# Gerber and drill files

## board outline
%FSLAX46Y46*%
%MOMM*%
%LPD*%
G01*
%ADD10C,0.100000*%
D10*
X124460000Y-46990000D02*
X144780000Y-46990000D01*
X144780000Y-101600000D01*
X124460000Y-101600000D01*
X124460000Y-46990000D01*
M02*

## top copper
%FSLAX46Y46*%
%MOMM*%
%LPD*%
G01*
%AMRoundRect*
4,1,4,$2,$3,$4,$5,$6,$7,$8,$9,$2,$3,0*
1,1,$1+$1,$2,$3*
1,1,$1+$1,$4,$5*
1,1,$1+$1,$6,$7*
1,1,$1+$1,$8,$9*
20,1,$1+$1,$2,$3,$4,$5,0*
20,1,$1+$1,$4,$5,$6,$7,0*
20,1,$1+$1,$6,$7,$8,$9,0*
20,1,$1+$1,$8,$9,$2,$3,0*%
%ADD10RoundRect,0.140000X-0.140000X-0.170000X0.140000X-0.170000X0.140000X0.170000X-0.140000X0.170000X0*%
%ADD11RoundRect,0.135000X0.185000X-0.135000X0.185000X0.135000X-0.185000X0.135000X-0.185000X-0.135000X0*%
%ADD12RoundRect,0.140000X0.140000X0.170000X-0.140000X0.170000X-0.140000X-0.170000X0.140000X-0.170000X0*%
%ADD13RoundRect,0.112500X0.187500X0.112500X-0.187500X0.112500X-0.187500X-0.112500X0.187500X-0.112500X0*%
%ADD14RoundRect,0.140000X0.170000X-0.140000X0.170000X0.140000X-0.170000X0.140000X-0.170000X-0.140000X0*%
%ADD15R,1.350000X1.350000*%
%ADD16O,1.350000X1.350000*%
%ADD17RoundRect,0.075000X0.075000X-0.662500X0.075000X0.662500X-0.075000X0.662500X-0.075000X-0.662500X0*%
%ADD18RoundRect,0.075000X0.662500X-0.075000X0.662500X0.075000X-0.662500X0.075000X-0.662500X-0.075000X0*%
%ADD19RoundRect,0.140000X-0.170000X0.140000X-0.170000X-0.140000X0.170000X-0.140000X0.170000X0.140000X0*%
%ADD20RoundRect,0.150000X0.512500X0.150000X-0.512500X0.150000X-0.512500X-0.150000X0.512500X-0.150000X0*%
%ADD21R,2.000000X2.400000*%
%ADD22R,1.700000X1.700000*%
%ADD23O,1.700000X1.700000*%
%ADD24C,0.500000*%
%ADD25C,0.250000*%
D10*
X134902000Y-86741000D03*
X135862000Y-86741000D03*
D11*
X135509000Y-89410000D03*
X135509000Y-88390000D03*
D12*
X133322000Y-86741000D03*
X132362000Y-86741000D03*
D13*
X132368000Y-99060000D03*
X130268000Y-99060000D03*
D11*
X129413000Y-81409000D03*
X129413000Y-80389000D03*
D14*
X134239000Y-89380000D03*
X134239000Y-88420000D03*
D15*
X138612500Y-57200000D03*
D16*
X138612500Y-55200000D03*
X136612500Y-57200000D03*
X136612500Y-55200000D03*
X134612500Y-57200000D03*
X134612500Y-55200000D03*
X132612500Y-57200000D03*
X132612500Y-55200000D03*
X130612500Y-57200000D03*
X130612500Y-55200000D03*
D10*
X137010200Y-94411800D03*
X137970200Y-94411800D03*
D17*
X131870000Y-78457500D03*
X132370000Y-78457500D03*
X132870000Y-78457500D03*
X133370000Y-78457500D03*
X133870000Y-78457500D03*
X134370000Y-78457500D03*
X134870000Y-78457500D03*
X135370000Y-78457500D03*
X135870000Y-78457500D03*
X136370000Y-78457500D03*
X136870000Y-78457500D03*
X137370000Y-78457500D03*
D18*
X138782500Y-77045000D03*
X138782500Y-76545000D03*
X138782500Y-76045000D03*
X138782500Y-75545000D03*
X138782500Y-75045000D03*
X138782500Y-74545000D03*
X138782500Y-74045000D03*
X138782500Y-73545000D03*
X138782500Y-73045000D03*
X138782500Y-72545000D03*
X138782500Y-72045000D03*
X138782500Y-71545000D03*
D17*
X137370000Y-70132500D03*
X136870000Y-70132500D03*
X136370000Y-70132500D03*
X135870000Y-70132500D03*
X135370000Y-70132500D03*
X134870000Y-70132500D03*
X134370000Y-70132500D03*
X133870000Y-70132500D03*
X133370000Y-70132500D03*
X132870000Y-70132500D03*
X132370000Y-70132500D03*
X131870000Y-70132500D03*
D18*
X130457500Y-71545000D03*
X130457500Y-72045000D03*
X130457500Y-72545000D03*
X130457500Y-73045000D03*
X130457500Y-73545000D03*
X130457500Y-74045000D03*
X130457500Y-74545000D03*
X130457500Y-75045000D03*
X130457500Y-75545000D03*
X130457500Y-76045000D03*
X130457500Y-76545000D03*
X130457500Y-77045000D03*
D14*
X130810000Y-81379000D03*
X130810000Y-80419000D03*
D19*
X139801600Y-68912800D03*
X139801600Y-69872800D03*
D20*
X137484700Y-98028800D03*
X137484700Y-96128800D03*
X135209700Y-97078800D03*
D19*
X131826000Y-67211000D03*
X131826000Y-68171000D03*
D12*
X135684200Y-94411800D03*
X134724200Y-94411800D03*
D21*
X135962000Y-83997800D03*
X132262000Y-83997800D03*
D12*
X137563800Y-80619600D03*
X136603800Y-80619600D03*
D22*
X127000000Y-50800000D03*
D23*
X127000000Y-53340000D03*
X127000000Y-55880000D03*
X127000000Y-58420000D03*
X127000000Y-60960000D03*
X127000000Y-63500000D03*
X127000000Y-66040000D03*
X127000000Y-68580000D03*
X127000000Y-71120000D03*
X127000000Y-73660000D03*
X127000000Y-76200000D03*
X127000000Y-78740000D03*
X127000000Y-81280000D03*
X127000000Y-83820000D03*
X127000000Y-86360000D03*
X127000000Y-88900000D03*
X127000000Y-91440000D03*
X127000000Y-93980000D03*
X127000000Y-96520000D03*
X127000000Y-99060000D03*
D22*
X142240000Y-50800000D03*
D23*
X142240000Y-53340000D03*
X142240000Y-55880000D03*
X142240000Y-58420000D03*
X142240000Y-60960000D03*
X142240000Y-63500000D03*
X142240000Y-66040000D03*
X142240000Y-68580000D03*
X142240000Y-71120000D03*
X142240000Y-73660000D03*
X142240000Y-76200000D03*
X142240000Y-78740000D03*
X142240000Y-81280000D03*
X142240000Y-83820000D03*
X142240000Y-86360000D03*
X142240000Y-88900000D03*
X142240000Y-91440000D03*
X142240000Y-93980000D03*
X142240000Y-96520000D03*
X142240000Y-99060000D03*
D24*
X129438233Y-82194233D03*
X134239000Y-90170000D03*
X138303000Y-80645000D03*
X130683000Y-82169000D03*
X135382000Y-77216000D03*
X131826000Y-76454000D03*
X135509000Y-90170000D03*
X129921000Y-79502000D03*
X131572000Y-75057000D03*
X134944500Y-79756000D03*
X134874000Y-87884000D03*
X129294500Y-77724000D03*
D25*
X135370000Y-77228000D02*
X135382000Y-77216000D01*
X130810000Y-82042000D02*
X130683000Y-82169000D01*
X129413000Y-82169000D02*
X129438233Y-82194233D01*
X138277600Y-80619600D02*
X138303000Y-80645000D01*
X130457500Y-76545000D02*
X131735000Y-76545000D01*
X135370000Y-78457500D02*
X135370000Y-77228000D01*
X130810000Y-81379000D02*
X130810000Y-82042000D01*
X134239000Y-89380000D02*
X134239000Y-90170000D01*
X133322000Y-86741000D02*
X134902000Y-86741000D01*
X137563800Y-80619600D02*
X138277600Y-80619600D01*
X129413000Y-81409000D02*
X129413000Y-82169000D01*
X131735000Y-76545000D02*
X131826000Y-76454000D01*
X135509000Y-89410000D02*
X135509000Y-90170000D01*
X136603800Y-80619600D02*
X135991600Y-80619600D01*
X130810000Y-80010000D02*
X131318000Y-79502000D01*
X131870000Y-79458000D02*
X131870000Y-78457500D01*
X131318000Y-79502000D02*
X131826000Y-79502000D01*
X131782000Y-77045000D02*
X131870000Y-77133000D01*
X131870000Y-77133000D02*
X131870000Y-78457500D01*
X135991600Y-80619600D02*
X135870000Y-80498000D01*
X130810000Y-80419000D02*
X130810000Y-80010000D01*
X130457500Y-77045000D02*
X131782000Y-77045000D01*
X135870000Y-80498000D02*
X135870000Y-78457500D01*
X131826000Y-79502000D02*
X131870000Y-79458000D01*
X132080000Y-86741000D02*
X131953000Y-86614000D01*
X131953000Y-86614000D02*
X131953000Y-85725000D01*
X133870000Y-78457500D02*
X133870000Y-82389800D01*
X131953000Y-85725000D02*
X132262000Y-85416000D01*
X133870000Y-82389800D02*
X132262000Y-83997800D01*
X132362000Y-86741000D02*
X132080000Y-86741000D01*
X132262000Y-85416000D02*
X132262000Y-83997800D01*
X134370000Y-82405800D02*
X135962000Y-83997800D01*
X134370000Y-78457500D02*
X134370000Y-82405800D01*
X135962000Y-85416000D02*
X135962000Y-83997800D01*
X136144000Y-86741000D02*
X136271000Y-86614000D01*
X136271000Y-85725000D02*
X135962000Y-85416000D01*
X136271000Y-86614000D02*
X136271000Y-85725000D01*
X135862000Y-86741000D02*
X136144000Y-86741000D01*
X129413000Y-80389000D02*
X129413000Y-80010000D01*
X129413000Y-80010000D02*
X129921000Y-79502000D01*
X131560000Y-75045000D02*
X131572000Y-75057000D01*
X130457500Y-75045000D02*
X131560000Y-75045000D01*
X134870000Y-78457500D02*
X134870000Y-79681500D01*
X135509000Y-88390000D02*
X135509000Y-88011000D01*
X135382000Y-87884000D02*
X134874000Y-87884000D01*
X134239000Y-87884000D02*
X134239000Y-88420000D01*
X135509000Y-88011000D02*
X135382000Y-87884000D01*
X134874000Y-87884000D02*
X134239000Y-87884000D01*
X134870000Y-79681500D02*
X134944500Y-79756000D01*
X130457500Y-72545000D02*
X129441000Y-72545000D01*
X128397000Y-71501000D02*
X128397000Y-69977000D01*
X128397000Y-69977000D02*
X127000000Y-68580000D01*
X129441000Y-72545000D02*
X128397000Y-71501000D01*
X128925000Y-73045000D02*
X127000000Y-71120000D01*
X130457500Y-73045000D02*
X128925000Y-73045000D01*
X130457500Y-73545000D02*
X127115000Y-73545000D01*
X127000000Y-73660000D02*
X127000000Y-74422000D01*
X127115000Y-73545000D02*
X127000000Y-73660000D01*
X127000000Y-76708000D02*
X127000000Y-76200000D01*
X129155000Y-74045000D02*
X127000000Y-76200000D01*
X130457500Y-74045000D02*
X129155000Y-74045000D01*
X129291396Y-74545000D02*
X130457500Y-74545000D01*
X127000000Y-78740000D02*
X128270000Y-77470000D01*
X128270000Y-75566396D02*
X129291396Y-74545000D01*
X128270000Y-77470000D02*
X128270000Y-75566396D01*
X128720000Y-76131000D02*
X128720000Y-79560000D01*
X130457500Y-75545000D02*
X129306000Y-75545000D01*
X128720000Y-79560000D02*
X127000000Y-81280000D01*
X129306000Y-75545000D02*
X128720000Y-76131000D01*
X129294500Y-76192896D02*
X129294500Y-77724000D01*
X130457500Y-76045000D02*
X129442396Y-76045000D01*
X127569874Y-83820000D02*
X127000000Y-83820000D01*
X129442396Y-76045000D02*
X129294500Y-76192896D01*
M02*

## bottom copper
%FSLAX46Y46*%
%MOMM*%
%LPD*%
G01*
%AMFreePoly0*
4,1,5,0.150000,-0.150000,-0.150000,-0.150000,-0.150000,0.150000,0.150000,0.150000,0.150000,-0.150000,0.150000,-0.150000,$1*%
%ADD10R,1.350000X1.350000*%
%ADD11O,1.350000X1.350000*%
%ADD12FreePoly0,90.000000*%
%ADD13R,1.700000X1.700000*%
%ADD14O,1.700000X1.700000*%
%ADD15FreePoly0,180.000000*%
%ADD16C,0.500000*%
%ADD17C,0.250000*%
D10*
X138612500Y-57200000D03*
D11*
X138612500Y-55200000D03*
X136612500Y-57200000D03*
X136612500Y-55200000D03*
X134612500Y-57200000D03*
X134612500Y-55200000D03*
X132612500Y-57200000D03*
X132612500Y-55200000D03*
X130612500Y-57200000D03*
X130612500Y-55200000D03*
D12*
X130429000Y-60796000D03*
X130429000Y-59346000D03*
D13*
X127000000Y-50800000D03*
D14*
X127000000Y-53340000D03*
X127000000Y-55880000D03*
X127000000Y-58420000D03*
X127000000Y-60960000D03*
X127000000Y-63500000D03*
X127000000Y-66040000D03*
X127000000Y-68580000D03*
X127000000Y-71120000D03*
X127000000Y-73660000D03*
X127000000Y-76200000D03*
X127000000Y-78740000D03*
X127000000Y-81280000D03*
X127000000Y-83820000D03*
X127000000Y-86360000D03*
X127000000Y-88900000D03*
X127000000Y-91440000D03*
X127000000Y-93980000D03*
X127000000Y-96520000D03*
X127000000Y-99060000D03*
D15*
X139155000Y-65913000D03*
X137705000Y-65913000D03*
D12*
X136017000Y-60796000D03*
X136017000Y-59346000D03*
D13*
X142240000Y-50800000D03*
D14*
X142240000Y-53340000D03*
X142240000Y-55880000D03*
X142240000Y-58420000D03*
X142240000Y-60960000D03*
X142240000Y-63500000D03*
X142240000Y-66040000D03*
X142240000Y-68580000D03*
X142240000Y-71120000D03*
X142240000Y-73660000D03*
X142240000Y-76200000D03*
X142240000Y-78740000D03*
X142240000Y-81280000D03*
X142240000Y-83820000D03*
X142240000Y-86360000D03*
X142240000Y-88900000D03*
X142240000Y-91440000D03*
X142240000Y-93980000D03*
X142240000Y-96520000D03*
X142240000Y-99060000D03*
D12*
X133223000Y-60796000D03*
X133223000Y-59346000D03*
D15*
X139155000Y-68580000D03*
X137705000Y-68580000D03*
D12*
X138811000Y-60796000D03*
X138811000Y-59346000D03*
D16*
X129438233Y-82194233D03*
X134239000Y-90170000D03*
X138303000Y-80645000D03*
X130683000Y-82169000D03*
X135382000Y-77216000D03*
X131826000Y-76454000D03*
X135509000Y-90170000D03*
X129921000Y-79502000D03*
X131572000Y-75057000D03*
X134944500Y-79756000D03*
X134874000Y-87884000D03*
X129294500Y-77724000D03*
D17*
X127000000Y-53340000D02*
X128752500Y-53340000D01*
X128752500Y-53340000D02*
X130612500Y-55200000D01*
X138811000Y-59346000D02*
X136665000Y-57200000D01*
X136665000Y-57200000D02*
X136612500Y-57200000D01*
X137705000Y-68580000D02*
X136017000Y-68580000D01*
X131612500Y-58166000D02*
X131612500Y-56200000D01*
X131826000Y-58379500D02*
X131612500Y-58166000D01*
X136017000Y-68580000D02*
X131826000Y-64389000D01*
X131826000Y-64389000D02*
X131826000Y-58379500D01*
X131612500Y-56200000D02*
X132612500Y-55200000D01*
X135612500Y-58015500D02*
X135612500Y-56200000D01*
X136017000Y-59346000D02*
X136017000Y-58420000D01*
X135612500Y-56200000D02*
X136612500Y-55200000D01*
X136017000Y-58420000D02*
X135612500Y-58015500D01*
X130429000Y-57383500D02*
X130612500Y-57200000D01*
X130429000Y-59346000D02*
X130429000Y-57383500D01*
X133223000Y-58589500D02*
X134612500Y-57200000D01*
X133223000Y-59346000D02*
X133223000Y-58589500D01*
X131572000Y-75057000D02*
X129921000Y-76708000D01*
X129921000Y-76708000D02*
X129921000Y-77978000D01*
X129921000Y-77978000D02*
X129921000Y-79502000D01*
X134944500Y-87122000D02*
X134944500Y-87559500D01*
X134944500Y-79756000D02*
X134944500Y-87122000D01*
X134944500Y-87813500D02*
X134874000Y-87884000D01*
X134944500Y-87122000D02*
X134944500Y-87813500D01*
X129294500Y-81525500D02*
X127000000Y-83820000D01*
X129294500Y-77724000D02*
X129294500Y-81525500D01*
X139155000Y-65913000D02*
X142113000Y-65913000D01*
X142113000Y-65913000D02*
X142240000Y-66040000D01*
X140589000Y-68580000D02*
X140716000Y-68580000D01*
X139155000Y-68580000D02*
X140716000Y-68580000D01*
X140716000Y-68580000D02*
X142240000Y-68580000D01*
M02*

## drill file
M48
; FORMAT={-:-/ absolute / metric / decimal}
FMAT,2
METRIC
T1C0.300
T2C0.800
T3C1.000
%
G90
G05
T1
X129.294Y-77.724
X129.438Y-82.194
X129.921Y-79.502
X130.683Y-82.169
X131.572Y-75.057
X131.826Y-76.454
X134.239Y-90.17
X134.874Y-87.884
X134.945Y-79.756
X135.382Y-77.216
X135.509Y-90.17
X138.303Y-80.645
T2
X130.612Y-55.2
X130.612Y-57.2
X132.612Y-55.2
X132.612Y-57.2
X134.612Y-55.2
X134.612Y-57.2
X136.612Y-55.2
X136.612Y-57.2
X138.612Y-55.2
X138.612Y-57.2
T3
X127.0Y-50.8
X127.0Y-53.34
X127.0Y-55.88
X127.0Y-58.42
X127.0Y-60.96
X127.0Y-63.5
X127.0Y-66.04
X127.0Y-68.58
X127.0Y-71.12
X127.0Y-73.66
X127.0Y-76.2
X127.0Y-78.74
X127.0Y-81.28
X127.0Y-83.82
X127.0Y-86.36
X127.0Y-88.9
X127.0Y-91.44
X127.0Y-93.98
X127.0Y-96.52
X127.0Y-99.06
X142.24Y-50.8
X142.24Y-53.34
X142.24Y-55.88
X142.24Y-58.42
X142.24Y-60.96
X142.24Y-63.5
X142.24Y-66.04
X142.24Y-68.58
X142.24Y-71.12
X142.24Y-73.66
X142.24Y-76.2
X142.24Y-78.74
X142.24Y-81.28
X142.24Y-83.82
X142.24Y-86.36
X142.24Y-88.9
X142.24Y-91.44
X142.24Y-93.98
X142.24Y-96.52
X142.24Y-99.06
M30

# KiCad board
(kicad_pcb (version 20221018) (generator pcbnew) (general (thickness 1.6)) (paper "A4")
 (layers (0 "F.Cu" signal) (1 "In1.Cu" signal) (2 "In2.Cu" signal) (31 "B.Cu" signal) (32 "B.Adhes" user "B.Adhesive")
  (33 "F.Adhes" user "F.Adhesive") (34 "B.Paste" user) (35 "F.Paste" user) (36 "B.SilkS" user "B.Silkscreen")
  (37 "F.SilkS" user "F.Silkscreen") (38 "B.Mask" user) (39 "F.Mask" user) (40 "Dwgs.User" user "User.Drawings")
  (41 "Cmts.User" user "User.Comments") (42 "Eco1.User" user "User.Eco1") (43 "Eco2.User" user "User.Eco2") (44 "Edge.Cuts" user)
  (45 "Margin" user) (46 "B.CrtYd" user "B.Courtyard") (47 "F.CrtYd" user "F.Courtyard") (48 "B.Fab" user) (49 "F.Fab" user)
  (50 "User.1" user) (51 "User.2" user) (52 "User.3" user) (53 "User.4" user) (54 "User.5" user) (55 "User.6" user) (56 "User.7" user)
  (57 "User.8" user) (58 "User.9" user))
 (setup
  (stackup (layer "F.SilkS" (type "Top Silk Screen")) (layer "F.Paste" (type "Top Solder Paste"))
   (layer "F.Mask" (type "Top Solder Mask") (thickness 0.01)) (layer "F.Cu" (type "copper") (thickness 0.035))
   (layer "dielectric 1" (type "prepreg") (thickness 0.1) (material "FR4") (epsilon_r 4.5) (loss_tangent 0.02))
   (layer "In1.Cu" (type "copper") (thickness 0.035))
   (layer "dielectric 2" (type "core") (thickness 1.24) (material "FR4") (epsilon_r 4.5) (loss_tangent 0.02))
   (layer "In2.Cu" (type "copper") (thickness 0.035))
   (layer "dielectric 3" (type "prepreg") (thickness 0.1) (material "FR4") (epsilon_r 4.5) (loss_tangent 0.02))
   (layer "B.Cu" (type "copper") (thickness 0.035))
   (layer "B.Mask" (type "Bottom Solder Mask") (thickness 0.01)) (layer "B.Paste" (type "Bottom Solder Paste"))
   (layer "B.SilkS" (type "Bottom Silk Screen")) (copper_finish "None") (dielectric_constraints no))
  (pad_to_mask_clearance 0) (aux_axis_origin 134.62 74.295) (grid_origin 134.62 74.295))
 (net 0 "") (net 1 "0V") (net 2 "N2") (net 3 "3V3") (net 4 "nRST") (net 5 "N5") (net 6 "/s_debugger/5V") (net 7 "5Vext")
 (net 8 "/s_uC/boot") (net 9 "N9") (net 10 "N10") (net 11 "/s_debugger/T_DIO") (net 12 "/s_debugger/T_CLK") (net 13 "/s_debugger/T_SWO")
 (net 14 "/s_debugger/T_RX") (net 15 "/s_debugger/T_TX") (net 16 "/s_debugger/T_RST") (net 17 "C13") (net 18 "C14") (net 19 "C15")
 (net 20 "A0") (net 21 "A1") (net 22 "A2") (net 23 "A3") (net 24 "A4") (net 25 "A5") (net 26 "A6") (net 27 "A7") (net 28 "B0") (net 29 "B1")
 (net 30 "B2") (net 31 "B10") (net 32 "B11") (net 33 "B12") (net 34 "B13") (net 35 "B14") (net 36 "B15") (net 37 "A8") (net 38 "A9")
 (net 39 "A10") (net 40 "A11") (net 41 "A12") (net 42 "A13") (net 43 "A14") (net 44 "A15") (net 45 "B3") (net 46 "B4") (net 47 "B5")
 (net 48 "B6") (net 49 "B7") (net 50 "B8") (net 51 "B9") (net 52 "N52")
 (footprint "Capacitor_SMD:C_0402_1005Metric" (layer "F.Cu") (at 135.382 86.741)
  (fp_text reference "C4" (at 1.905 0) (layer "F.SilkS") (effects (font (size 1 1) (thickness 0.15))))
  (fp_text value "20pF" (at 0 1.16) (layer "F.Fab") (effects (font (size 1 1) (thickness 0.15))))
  (pad "1" smd roundrect (at -0.48 0) (size 0.56 0.62) (layers "F.Cu" "F.Paste" "F.Mask") (roundrect_rratio 0.25) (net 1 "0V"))
  (pad "2" smd roundrect (at 0.48 0) (size 0.56 0.62) (layers "F.Cu" "F.Paste" "F.Mask") (roundrect_rratio 0.25) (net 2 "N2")))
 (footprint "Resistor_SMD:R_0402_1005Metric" (layer "F.Cu") (at 135.509 88.9 90)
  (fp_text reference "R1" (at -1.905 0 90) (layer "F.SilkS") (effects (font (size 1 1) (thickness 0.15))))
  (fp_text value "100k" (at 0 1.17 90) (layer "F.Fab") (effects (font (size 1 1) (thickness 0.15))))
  (pad "1" smd roundrect (at -0.51 0 90) (size 0.54 0.64) (layers "F.Cu" "F.Paste" "F.Mask") (roundrect_rratio 0.25) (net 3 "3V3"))
  (pad "2" smd roundrect (at 0.51 0 90) (size 0.54 0.64) (layers "F.Cu" "F.Paste" "F.Mask") (roundrect_rratio 0.25) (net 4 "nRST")))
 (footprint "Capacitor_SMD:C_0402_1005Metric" (layer "F.Cu") (at 132.842 86.741 180)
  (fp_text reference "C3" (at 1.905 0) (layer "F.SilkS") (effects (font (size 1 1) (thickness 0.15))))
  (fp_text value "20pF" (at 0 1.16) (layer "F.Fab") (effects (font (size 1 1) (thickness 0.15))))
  (pad "1" smd roundrect (at -0.48 0 180) (size 0.56 0.62) (layers "F.Cu" "F.Paste" "F.Mask") (roundrect_rratio 0.25) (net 1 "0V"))
  (pad "2" smd roundrect (at 0.48 0 180) (size 0.56 0.62) (layers "F.Cu" "F.Paste" "F.Mask") (roundrect_rratio 0.25) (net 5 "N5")))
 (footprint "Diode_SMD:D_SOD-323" (layer "F.Cu") (at 131.318 99.06 180)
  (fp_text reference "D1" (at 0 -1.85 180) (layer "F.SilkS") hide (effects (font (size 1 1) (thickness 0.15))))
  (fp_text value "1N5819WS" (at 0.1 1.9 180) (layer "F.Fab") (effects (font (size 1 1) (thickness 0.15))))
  (pad "1" smd roundrect (at -1.05 0 180) (size 0.6 0.45) (layers "F.Cu" "F.Paste" "F.Mask") (roundrect_rratio 0.25)
   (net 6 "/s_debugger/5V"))
  (pad "2" smd roundrect (at 1.05 0 180) (size 0.6 0.45) (layers "F.Cu" "F.Paste" "F.Mask") (roundrect_rratio 0.25) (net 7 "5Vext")))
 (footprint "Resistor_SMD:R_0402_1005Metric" (layer "F.Cu") (at 129.413 80.899 90)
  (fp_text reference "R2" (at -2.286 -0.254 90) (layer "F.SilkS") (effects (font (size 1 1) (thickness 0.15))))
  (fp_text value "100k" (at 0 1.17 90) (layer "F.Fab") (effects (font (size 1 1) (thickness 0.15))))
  (pad "1" smd roundrect (at -0.51 0 90) (size 0.54 0.64) (layers "F.Cu" "F.Paste" "F.Mask") (roundrect_rratio 0.25) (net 1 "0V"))
  (pad "2" smd roundrect (at 0.51 0 90) (size 0.54 0.64) (layers "F.Cu" "F.Paste" "F.Mask") (roundrect_rratio 0.25) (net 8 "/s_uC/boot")))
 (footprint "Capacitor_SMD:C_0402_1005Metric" (layer "F.Cu") (at 134.239 88.9 90)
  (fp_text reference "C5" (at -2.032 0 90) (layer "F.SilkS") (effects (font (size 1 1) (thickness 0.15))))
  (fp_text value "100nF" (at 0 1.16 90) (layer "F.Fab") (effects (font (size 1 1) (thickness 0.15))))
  (pad "1" smd roundrect (at -0.48 0 90) (size 0.56 0.62) (layers "F.Cu" "F.Paste" "F.Mask") (roundrect_rratio 0.25) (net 1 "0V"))
  (pad "2" smd roundrect (at 0.48 0 90) (size 0.56 0.62) (layers "F.Cu" "F.Paste" "F.Mask") (roundrect_rratio 0.25) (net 4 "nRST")))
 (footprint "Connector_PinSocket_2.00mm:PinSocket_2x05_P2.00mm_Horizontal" (layer "F.Cu") (at 138.6125 57.2 -90)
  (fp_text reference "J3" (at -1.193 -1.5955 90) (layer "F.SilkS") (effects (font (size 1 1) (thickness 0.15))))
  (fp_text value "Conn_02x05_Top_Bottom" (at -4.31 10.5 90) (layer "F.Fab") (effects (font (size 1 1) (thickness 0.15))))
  (pad "1" thru_hole rect (at 0 0 270) (size 1.35 1.35) (drill 0.8) (layers "*.Cu" "*.Mask") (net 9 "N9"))
  (pad "2" thru_hole oval (at -2 0 270) (size 1.35 1.35) (drill 0.8) (layers "*.Cu" "*.Mask") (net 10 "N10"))
  (pad "3" thru_hole oval (at 0 2 270) (size 1.35 1.35) (drill 0.8) (layers "*.Cu" "*.Mask") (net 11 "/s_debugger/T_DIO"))
  (pad "4" thru_hole oval (at -2 2 270) (size 1.35 1.35) (drill 0.8) (layers "*.Cu" "*.Mask") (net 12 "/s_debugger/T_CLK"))
  (pad "5" thru_hole oval (at 0 4 270) (size 1.35 1.35) (drill 0.8) (layers "*.Cu" "*.Mask") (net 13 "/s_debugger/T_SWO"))
  (pad "6" thru_hole oval (at -2 4 270) (size 1.35 1.35) (drill 0.8) (layers "*.Cu" "*.Mask") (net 1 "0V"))
  (pad "7" thru_hole oval (at 0 6 270) (size 1.35 1.35) (drill 0.8) (layers "*.Cu" "*.Mask") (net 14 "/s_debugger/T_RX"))
  (pad "8" thru_hole oval (at -2 6 270) (size 1.35 1.35) (drill 0.8) (layers "*.Cu" "*.Mask") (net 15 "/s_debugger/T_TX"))
  (pad "9" thru_hole oval (at 0 8 270) (size 1.35 1.35) (drill 0.8) (layers "*.Cu" "*.Mask") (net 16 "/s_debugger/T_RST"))
  (pad "10" thru_hole oval (at -2 8 270) (size 1.35 1.35) (drill 0.8) (layers "*.Cu" "*.Mask") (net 3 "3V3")))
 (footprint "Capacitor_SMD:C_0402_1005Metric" (layer "F.Cu") (at 137.4902 94.4118)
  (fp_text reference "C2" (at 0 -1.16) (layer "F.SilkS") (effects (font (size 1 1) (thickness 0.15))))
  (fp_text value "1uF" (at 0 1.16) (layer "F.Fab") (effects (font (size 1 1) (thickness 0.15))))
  (pad "1" smd roundrect (at -0.48 0) (size 0.56 0.62) (layers "F.Cu" "F.Paste" "F.Mask") (roundrect_rratio 0.25) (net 1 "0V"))
  (pad "2" smd roundrect (at 0.48 0) (size 0.56 0.62) (layers "F.Cu" "F.Paste" "F.Mask") (roundrect_rratio 0.25) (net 3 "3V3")))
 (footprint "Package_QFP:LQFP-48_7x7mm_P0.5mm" (layer "F.Cu") (at 134.62 74.295 90)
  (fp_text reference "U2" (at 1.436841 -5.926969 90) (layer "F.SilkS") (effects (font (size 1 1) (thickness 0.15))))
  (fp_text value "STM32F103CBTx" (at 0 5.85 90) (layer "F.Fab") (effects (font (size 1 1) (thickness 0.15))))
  (pad "1" smd roundrect (at -4.1625 -2.75 90) (size 1.475 0.3) (layers "F.Cu" "F.Paste" "F.Mask") (roundrect_rratio 0.25) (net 3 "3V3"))
  (pad "2" smd roundrect (at -4.1625 -2.25 90) (size 1.475 0.3) (layers "F.Cu" "F.Paste" "F.Mask") (roundrect_rratio 0.25) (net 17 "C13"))
  (pad "3" smd roundrect (at -4.1625 -1.75 90) (size 1.475 0.3) (layers "F.Cu" "F.Paste" "F.Mask") (roundrect_rratio 0.25) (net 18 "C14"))
  (pad "4" smd roundrect (at -4.1625 -1.25 90) (size 1.475 0.3) (layers "F.Cu" "F.Paste" "F.Mask") (roundrect_rratio 0.25) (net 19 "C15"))
  (pad "5" smd roundrect (at -4.1625 -0.75 90) (size 1.475 0.3) (layers "F.Cu" "F.Paste" "F.Mask") (roundrect_rratio 0.25) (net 5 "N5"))
  (pad "6" smd roundrect (at -4.1625 -0.25 90) (size 1.475 0.3) (layers "F.Cu" "F.Paste" "F.Mask") (roundrect_rratio 0.25) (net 2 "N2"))
  (pad "7" smd roundrect (at -4.1625 0.25 90) (size 1.475 0.3) (layers "F.Cu" "F.Paste" "F.Mask") (roundrect_rratio 0.25) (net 4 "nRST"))
  (pad "8" smd roundrect (at -4.1625 0.75 90) (size 1.475 0.3) (layers "F.Cu" "F.Paste" "F.Mask") (roundrect_rratio 0.25) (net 1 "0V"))
  (pad "9" smd roundrect (at -4.1625 1.25 90) (size 1.475 0.3) (layers "F.Cu" "F.Paste" "F.Mask") (roundrect_rratio 0.25) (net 3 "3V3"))
  (pad "10" smd roundrect (at -4.1625 1.75 90) (size 1.475 0.3) (layers "F.Cu" "F.Paste" "F.Mask") (roundrect_rratio 0.25) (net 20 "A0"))
  (pad "11" smd roundrect (at -4.1625 2.25 90) (size 1.475 0.3) (layers "F.Cu" "F.Paste" "F.Mask") (roundrect_rratio 0.25) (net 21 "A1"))
  (pad "12" smd roundrect (at -4.1625 2.75 90) (size 1.475 0.3) (layers "F.Cu" "F.Paste" "F.Mask") (roundrect_rratio 0.25) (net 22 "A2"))
  (pad "13" smd roundrect (at -2.75 4.1625 90) (size 0.3 1.475) (layers "F.Cu" "F.Paste" "F.Mask") (roundrect_rratio 0.25) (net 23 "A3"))
  (pad "14" smd roundrect (at -2.25 4.1625 90) (size 0.3 1.475) (layers "F.Cu" "F.Paste" "F.Mask") (roundrect_rratio 0.25) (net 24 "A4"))
  (pad "15" smd roundrect (at -1.75 4.1625 90) (size 0.3 1.475) (layers "F.Cu" "F.Paste" "F.Mask") (roundrect_rratio 0.25) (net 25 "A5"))
  (pad "16" smd roundrect (at -1.25 4.1625 90) (size 0.3 1.475) (layers "F.Cu" "F.Paste" "F.Mask") (roundrect_rratio 0.25) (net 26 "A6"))
  (pad "17" smd roundrect (at -0.75 4.1625 90) (size 0.3 1.475) (layers "F.Cu" "F.Paste" "F.Mask") (roundrect_rratio 0.25) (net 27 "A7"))
  (pad "18" smd roundrect (at -0.25 4.1625 90) (size 0.3 1.475) (layers "F.Cu" "F.Paste" "F.Mask") (roundrect_rratio 0.25) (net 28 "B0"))
  (pad "19" smd roundrect (at 0.25 4.1625 90) (size 0.3 1.475) (layers "F.Cu" "F.Paste" "F.Mask") (roundrect_rratio 0.25) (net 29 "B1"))
  (pad "20" smd roundrect (at 0.75 4.1625 90) (size 0.3 1.475) (layers "F.Cu" "F.Paste" "F.Mask") (roundrect_rratio 0.25) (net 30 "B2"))
  (pad "21" smd roundrect (at 1.25 4.1625 90) (size 0.3 1.475) (layers "F.Cu" "F.Paste" "F.Mask") (roundrect_rratio 0.25) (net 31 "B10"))
  (pad "22" smd roundrect (at 1.75 4.1625 90) (size 0.3 1.475) (layers "F.Cu" "F.Paste" "F.Mask") (roundrect_rratio 0.25) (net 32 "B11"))
  (pad "23" smd roundrect (at 2.25 4.1625 90) (size 0.3 1.475) (layers "F.Cu" "F.Paste" "F.Mask") (roundrect_rratio 0.25) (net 1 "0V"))
  (pad "24" smd roundrect (at 2.75 4.1625 90) (size 0.3 1.475) (layers "F.Cu" "F.Paste" "F.Mask") (roundrect_rratio 0.25) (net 3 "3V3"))
  (pad "25" smd roundrect (at 4.1625 2.75 90) (size 1.475 0.3) (layers "F.Cu" "F.Paste" "F.Mask") (roundrect_rratio 0.25) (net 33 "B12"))
  (pad "26" smd roundrect (at 4.1625 2.25 90) (size 1.475 0.3) (layers "F.Cu" "F.Paste" "F.Mask") (roundrect_rratio 0.25) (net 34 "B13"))
  (pad "27" smd roundrect (at 4.1625 1.75 90) (size 1.475 0.3) (layers "F.Cu" "F.Paste" "F.Mask") (roundrect_rratio 0.25) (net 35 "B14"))
  (pad "28" smd roundrect (at 4.1625 1.25 90) (size 1.475 0.3) (layers "F.Cu" "F.Paste" "F.Mask") (roundrect_rratio 0.25) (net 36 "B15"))
  (pad "29" smd roundrect (at 4.1625 0.75 90) (size 1.475 0.3) (layers "F.Cu" "F.Paste" "F.Mask") (roundrect_rratio 0.25) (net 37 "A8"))
  (pad "30" smd roundrect (at 4.1625 0.25 90) (size 1.475 0.3) (layers "F.Cu" "F.Paste" "F.Mask") (roundrect_rratio 0.25) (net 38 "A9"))
  (pad "31" smd roundrect (at 4.1625 -0.25 90) (size 1.475 0.3) (layers "F.Cu" "F.Paste" "F.Mask") (roundrect_rratio 0.25) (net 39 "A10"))
  (pad "32" smd roundrect (at 4.1625 -0.75 90) (size 1.475 0.3) (layers "F.Cu" "F.Paste" "F.Mask") (roundrect_rratio 0.25) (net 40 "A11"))
  (pad "33" smd roundrect (at 4.1625 -1.25 90) (size 1.475 0.3) (layers "F.Cu" "F.Paste" "F.Mask") (roundrect_rratio 0.25) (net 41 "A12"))
  (pad "34" smd roundrect (at 4.1625 -1.75 90) (size 1.475 0.3) (layers "F.Cu" "F.Paste" "F.Mask") (roundrect_rratio 0.25) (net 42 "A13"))
  (pad "35" smd roundrect (at 4.1625 -2.25 90) (size 1.475 0.3) (layers "F.Cu" "F.Paste" "F.Mask") (roundrect_rratio 0.25) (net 1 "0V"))
  (pad "36" smd roundrect (at 4.1625 -2.75 90) (size 1.475 0.3) (layers "F.Cu" "F.Paste" "F.Mask") (roundrect_rratio 0.25) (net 3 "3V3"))
  (pad "37" smd roundrect (at 2.75 -4.1625 90) (size 0.3 1.475) (layers "F.Cu" "F.Paste" "F.Mask") (roundrect_rratio 0.25) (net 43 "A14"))
  (pad "38" smd roundrect (at 2.25 -4.1625 90) (size 0.3 1.475) (layers "F.Cu" "F.Paste" "F.Mask") (roundrect_rratio 0.25) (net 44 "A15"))
  (pad "39" smd roundrect (at 1.75 -4.1625 90) (size 0.3 1.475) (layers "F.Cu" "F.Paste" "F.Mask") (roundrect_rratio 0.25) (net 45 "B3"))
  (pad "40" smd roundrect (at 1.25 -4.1625 90) (size 0.3 1.475) (layers "F.Cu" "F.Paste" "F.Mask") (roundrect_rratio 0.25) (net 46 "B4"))
  (pad "41" smd roundrect (at 0.75 -4.1625 90) (size 0.3 1.475) (layers "F.Cu" "F.Paste" "F.Mask") (roundrect_rratio 0.25) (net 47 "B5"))
  (pad "42" smd roundrect (at 0.25 -4.1625 90) (size 0.3 1.475) (layers "F.Cu" "F.Paste" "F.Mask") (roundrect_rratio 0.25) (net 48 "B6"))
  (pad "43" smd roundrect (at -0.25 -4.1625 90) (size 0.3 1.475) (layers "F.Cu" "F.Paste" "F.Mask") (roundrect_rratio 0.25) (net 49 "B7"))
  (pad "44" smd roundrect (at -0.75 -4.1625 90) (size 0.3 1.475) (layers "F.Cu" "F.Paste" "F.Mask") (roundrect_rratio 0.25)
   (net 8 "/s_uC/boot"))
  (pad "45" smd roundrect (at -1.25 -4.1625 90) (size 0.3 1.475) (layers "F.Cu" "F.Paste" "F.Mask") (roundrect_rratio 0.25) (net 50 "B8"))
  (pad "46" smd roundrect (at -1.75 -4.1625 90) (size 0.3 1.475) (layers "F.Cu" "F.Paste" "F.Mask") (roundrect_rratio 0.25) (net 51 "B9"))
  (pad "47" smd roundrect (at -2.25 -4.1625 90) (size 0.3 1.475) (layers "F.Cu" "F.Paste" "F.Mask") (roundrect_rratio 0.25) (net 1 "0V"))
  (pad "48" smd roundrect (at -2.75 -4.1625 90) (size 0.3 1.475) (layers "F.Cu" "F.Paste" "F.Mask") (roundrect_rratio 0.25) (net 3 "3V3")))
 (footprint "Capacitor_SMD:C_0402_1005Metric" (layer "F.Cu") (at 130.81 80.899 90)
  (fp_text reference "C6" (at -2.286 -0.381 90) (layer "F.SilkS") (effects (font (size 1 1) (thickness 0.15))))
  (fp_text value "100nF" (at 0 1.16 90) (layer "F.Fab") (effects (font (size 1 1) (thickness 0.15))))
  (pad "1" smd roundrect (at -0.48 0 90) (size 0.56 0.62) (layers "F.Cu" "F.Paste" "F.Mask") (roundrect_rratio 0.25) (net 1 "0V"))
  (pad "2" smd roundrect (at 0.48 0 90) (size 0.56 0.62) (layers "F.Cu" "F.Paste" "F.Mask") (roundrect_rratio 0.25) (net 3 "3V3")))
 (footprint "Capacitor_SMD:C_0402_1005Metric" (layer "F.Cu") (at 139.8016 69.3928 -90)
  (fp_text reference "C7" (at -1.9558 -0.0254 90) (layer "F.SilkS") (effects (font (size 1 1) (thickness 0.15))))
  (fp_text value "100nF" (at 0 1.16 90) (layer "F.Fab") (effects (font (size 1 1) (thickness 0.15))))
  (pad "1" smd roundrect (at -0.48 0 270) (size 0.56 0.62) (layers "F.Cu" "F.Paste" "F.Mask") (roundrect_rratio 0.25) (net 1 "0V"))
  (pad "2" smd roundrect (at 0.48 0 270) (size 0.56 0.62) (layers "F.Cu" "F.Paste" "F.Mask") (roundrect_rratio 0.25) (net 3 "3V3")))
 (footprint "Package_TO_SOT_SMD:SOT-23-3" (layer "F.Cu") (at 136.3472 97.0788 180)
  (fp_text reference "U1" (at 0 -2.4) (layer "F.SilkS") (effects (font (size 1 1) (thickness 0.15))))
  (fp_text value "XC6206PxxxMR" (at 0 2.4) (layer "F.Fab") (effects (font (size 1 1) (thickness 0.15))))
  (pad "1" smd roundrect (at -1.1375 -0.95 180) (size 1.325 0.6) (layers "F.Cu" "F.Paste" "F.Mask") (roundrect_rratio 0.25) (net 1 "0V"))
  (pad "2" smd roundrect (at -1.1375 0.95 180) (size 1.325 0.6) (layers "F.Cu" "F.Paste" "F.Mask") (roundrect_rratio 0.25) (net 3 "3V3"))
  (pad "3" smd roundrect (at 1.1375 0 180) (size 1.325 0.6) (layers "F.Cu" "F.Paste" "F.Mask") (roundrect_rratio 0.25)
   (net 6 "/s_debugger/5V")))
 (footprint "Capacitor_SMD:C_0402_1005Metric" (layer "F.Cu") (at 131.826 67.691 -90)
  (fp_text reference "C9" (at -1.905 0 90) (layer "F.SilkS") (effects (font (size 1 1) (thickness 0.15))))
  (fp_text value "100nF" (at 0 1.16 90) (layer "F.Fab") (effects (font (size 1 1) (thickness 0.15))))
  (pad "1" smd roundrect (at -0.48 0 270) (size 0.56 0.62) (layers "F.Cu" "F.Paste" "F.Mask") (roundrect_rratio 0.25) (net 1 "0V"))
  (pad "2" smd roundrect (at 0.48 0 270) (size 0.56 0.62) (layers "F.Cu" "F.Paste" "F.Mask") (roundrect_rratio 0.25) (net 3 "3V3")))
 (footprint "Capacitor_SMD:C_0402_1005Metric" (layer "F.Cu") (at 135.2042 94.4118 180)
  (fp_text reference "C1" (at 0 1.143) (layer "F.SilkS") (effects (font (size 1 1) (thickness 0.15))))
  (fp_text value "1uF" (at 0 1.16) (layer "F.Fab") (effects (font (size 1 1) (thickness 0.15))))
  (pad "1" smd roundrect (at -0.48 0 180) (size 0.56 0.62) (layers "F.Cu" "F.Paste" "F.Mask") (roundrect_rratio 0.25) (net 1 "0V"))
  (pad "2" smd roundrect (at 0.48 0 180) (size 0.56 0.62) (layers "F.Cu" "F.Paste" "F.Mask") (roundrect_rratio 0.25)
   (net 6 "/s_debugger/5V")))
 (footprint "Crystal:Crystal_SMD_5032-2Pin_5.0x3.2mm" (layer "F.Cu") (at 134.112 83.9978 180)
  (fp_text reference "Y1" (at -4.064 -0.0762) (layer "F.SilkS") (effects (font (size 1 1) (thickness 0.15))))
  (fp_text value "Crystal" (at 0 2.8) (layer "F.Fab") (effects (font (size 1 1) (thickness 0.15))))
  (pad "1" smd rect (at -1.85 0 180) (size 2 2.4) (layers "F.Cu" "F.Paste" "F.Mask") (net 2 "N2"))
  (pad "2" smd rect (at 1.85 0 180) (size 2 2.4) (layers "F.Cu" "F.Paste" "F.Mask") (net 5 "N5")))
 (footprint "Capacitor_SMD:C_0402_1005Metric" (layer "F.Cu") (at 137.0838 80.6196 180)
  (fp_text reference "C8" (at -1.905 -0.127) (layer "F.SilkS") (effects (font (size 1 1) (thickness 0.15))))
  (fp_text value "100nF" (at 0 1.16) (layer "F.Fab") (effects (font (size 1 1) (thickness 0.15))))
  (pad "1" smd roundrect (at -0.48 0 180) (size 0.56 0.62) (layers "F.Cu" "F.Paste" "F.Mask") (roundrect_rratio 0.25) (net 1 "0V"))
  (pad "2" smd roundrect (at 0.48 0 180) (size 0.56 0.62) (layers "F.Cu" "F.Paste" "F.Mask") (roundrect_rratio 0.25) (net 3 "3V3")))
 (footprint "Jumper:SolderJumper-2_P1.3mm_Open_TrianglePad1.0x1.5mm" (layer "B.Cu") (at 130.429 60.071 90)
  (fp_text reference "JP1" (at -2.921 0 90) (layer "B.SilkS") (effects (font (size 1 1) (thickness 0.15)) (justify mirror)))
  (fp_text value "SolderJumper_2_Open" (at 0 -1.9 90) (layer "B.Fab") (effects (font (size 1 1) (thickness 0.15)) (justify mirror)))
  (pad "1" smd custom (at -0.725 0 90) (size 0.3 0.3) (layers "B.Cu" "B.Mask") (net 4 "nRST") (zone_connect 2)
   (options (clearance outline) (anchor rect)) (primitives))
  (pad "2" smd custom (at 0.725 0 90) (size 0.3 0.3) (layers "B.Cu" "B.Mask") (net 16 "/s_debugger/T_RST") (zone_connect 2)
   (options (clearance outline) (anchor rect)) (primitives)))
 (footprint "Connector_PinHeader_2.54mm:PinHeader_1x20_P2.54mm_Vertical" (layer "B.Cu") (at 127 50.8 180)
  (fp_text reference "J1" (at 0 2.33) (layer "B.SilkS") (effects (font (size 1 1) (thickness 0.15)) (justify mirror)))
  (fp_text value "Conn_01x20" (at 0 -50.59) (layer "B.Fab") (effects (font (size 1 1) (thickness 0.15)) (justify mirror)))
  (pad "1" thru_hole rect (at 0 0 180) (size 1.7 1.7) (drill 1) (layers "*.Cu" "*.Mask") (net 7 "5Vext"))
  (pad "2" thru_hole oval (at 0 -2.54 180) (size 1.7 1.7) (drill 1) (layers "*.Cu" "*.Mask") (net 3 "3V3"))
  (pad "3" thru_hole oval (at 0 -5.08 180) (size 1.7 1.7) (drill 1) (layers "*.Cu" "*.Mask") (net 1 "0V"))
  (pad "4" thru_hole oval (at 0 -7.62 180) (size 1.7 1.7) (drill 1) (layers "*.Cu" "*.Mask") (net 4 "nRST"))
  (pad "5" thru_hole oval (at 0 -10.16 180) (size 1.7 1.7) (drill 1) (layers "*.Cu" "*.Mask") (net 28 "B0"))
  (pad "6" thru_hole oval (at 0 -12.7 180) (size 1.7 1.7) (drill 1) (layers "*.Cu" "*.Mask") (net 29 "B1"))
  (pad "7" thru_hole oval (at 0 -15.24 180) (size 1.7 1.7) (drill 1) (layers "*.Cu" "*.Mask") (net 30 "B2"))
  (pad "8" thru_hole oval (at 0 -17.78 180) (size 1.7 1.7) (drill 1) (layers "*.Cu" "*.Mask") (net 45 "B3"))
  (pad "9" thru_hole oval (at 0 -20.32 180) (size 1.7 1.7) (drill 1) (layers "*.Cu" "*.Mask") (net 46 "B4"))
  (pad "10" thru_hole oval (at 0 -22.86 180) (size 1.7 1.7) (drill 1) (layers "*.Cu" "*.Mask") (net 47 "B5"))
  (pad "11" thru_hole oval (at 0 -25.4 180) (size 1.7 1.7) (drill 1) (layers "*.Cu" "*.Mask") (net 48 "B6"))
  (pad "12" thru_hole oval (at 0 -27.94 180) (size 1.7 1.7) (drill 1) (layers "*.Cu" "*.Mask") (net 49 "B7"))
  (pad "13" thru_hole oval (at 0 -30.48 180) (size 1.7 1.7) (drill 1) (layers "*.Cu" "*.Mask") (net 50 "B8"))
  (pad "14" thru_hole oval (at 0 -33.02 180) (size 1.7 1.7) (drill 1) (layers "*.Cu" "*.Mask") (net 51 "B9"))
  (pad "15" thru_hole oval (at 0 -35.56 180) (size 1.7 1.7) (drill 1) (layers "*.Cu" "*.Mask") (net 31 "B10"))
  (pad "16" thru_hole oval (at 0 -38.1 180) (size 1.7 1.7) (drill 1) (layers "*.Cu" "*.Mask") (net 32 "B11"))
  (pad "17" thru_hole oval (at 0 -40.64 180) (size 1.7 1.7) (drill 1) (layers "*.Cu" "*.Mask") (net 33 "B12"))
  (pad "18" thru_hole oval (at 0 -43.18 180) (size 1.7 1.7) (drill 1) (layers "*.Cu" "*.Mask") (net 34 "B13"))
  (pad "19" thru_hole oval (at 0 -45.72 180) (size 1.7 1.7) (drill 1) (layers "*.Cu" "*.Mask") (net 35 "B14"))
  (pad "20" thru_hole oval (at 0 -48.26 180) (size 1.7 1.7) (drill 1) (layers "*.Cu" "*.Mask") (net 36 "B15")))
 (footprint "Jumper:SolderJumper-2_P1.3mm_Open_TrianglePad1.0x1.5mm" (layer "B.Cu") (at 138.43 65.913 180)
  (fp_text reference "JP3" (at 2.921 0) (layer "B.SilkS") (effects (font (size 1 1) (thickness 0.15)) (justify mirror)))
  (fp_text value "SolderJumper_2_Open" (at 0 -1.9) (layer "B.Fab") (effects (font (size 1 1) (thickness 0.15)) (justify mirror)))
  (pad "1" smd custom (at -0.725 0 180) (size 0.3 0.3) (layers "B.Cu" "B.Mask") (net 22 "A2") (zone_connect 2)
   (options (clearance outline) (anchor rect)) (primitives))
  (pad "2" smd custom (at 0.725 0 180) (size 0.3 0.3) (layers "B.Cu" "B.Mask") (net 14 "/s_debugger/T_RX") (zone_connect 2)
   (options (clearance outline) (anchor rect)) (primitives)))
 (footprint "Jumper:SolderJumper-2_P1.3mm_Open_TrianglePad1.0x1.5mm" (layer "B.Cu") (at 136.017 60.071 90)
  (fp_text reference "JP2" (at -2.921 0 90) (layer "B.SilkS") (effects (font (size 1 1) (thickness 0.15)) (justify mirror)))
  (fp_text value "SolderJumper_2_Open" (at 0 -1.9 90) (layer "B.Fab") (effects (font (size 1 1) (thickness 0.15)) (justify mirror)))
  (pad "1" smd custom (at -0.725 0 90) (size 0.3 0.3) (layers "B.Cu" "B.Mask") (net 43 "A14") (zone_connect 2)
   (options (clearance outline) (anchor rect)) (primitives))
  (pad "2" smd custom (at 0.725 0 90) (size 0.3 0.3) (layers "B.Cu" "B.Mask") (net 12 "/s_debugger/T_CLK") (zone_connect 2)
   (options (clearance outline) (anchor rect)) (primitives)))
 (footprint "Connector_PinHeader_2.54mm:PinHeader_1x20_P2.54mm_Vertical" (layer "B.Cu") (at 142.24 50.8 180)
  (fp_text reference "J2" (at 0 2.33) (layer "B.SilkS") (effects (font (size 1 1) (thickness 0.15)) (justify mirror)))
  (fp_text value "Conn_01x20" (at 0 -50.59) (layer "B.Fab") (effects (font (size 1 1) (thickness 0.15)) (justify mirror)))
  (pad "1" thru_hole rect (at 0 0 180) (size 1.7 1.7) (drill 1) (layers "*.Cu" "*.Mask") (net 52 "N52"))
  (pad "2" thru_hole oval (at 0 -2.54 180) (size 1.7 1.7) (drill 1) (layers "*.Cu" "*.Mask") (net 17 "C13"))
  (pad "3" thru_hole oval (at 0 -5.08 180) (size 1.7 1.7) (drill 1) (layers "*.Cu" "*.Mask") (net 18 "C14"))
  (pad "4" thru_hole oval (at 0 -7.62 180) (size 1.7 1.7) (drill 1) (layers "*.Cu" "*.Mask") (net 19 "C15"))
  (pad "5" thru_hole oval (at 0 -10.16 180) (size 1.7 1.7) (drill 1) (layers "*.Cu" "*.Mask") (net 20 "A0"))
  (pad "6" thru_hole oval (at 0 -12.7 180) (size 1.7 1.7) (drill 1) (layers "*.Cu" "*.Mask") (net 21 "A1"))
  (pad "7" thru_hole oval (at 0 -15.24 180) (size 1.7 1.7) (drill 1) (layers "*.Cu" "*.Mask") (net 22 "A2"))
  (pad "8" thru_hole oval (at 0 -17.78 180) (size 1.7 1.7) (drill 1) (layers "*.Cu" "*.Mask") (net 23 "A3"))
  (pad "9" thru_hole oval (at 0 -20.32 180) (size 1.7 1.7) (drill 1) (layers "*.Cu" "*.Mask") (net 24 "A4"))
  (pad "10" thru_hole oval (at 0 -22.86 180) (size 1.7 1.7) (drill 1) (layers "*.Cu" "*.Mask") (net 25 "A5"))
  (pad "11" thru_hole oval (at 0 -25.4 180) (size 1.7 1.7) (drill 1) (layers "*.Cu" "*.Mask") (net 26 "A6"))
  (pad "12" thru_hole oval (at 0 -27.94 180) (size 1.7 1.7) (drill 1) (layers "*.Cu" "*.Mask") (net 27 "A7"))
  (pad "13" thru_hole oval (at 0 -30.48 180) (size 1.7 1.7) (drill 1) (layers "*.Cu" "*.Mask") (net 37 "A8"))
  (pad "14" thru_hole oval (at 0 -33.02 180) (size 1.7 1.7) (drill 1) (layers "*.Cu" "*.Mask") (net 38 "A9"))
  (pad "15" thru_hole oval (at 0 -35.56 180) (size 1.7 1.7) (drill 1) (layers "*.Cu" "*.Mask") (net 39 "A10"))
  (pad "16" thru_hole oval (at 0 -38.1 180) (size 1.7 1.7) (drill 1) (layers "*.Cu" "*.Mask") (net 40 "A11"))
  (pad "17" thru_hole oval (at 0 -40.64 180) (size 1.7 1.7) (drill 1) (layers "*.Cu" "*.Mask") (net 41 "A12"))
  (pad "18" thru_hole oval (at 0 -43.18 180) (size 1.7 1.7) (drill 1) (layers "*.Cu" "*.Mask") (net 42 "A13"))
  (pad "19" thru_hole oval (at 0 -45.72 180) (size 1.7 1.7) (drill 1) (layers "*.Cu" "*.Mask") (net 43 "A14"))
  (pad "20" thru_hole oval (at 0 -48.26 180) (size 1.7 1.7) (drill 1) (layers "*.Cu" "*.Mask") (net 44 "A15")))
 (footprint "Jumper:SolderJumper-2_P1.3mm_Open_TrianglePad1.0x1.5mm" (layer "B.Cu") (at 133.223 60.071 90)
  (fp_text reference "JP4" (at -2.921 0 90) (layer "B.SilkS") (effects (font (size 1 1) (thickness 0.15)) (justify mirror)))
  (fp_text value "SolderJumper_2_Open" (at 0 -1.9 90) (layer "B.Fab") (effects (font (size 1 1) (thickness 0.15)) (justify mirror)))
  (pad "1" smd custom (at -0.725 0 90) (size 0.3 0.3) (layers "B.Cu" "B.Mask") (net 37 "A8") (zone_connect 2)
   (options (clearance outline) (anchor rect)) (primitives))
  (pad "2" smd custom (at 0.725 0 90) (size 0.3 0.3) (layers "B.Cu" "B.Mask") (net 13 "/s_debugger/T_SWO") (zone_connect 2)
   (options (clearance outline) (anchor rect)) (primitives)))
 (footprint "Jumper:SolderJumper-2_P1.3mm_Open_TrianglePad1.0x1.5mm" (layer "B.Cu") (at 138.43 68.58 180)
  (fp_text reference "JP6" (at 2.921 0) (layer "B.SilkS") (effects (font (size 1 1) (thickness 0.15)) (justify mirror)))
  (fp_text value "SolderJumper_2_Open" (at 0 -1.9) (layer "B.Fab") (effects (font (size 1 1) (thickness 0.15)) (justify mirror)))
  (pad "1" smd custom (at -0.725 0 180) (size 0.3 0.3) (layers "B.Cu" "B.Mask") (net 23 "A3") (zone_connect 2)
   (options (clearance outline) (anchor rect)) (primitives))
  (pad "2" smd custom (at 0.725 0 180) (size 0.3 0.3) (layers "B.Cu" "B.Mask") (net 15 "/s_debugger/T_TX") (zone_connect 2)
   (options (clearance outline) (anchor rect)) (primitives)))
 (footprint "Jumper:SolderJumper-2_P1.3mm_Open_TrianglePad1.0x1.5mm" (layer "B.Cu") (at 138.811 60.071 90)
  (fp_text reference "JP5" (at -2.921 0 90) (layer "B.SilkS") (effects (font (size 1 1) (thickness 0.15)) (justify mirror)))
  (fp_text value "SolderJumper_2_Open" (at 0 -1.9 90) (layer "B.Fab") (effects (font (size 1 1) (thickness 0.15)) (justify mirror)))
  (pad "1" smd custom (at -0.725 0 90) (size 0.3 0.3) (layers "B.Cu" "B.Mask") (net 42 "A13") (zone_connect 2)
   (options (clearance outline) (anchor rect)) (primitives))
  (pad "2" smd custom (at 0.725 0 90) (size 0.3 0.3) (layers "B.Cu" "B.Mask") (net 11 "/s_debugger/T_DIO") (zone_connect 2)
   (options (clearance outline) (anchor rect)) (primitives)))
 (gr_rect (start 124.46 46.99) (end 144.78 101.6) (stroke (width 0.1) (type default)) (fill none) (layer "Edge.Cuts"))
 (segment (start 135.37 77.228) (end 135.382 77.216) (width 0.25) (layer "F.Cu") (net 1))
 (segment (start 130.81 82.042) (end 130.683 82.169) (width 0.25) (layer "F.Cu") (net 1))
 (segment (start 129.413 82.169) (end 129.438233 82.194233) (width 0.25) (layer "F.Cu") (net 1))
 (segment (start 138.2776 80.6196) (end 138.303 80.645) (width 0.25) (layer "F.Cu") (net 1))
 (segment (start 130.4575 76.545) (end 131.735 76.545) (width 0.25) (layer "F.Cu") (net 1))
 (segment (start 135.37 78.4575) (end 135.37 77.228) (width 0.25) (layer "F.Cu") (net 1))
 (segment (start 130.81 81.379) (end 130.81 82.042) (width 0.25) (layer "F.Cu") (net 1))
 (segment (start 134.239 89.38) (end 134.239 90.17) (width 0.25) (layer "F.Cu") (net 1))
 (segment (start 133.322 86.741) (end 134.902 86.741) (width 0.25) (layer "F.Cu") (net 1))
 (segment (start 137.5638 80.6196) (end 138.2776 80.6196) (width 0.25) (layer "F.Cu") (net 1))
 (segment (start 129.413 81.409) (end 129.413 82.169) (width 0.25) (layer "F.Cu") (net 1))
 (segment (start 131.735 76.545) (end 131.826 76.454) (width 0.25) (layer "F.Cu") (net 1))
 (via (at 129.438233 82.194233) (size 0.5) (drill 0.3) (layers "F.Cu" "B.Cu") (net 1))
 (via (at 134.239 90.17) (size 0.5) (drill 0.3) (layers "F.Cu" "B.Cu") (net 1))
 (via (at 138.303 80.645) (size 0.5) (drill 0.3) (layers "F.Cu" "B.Cu") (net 1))
 (via (at 130.683 82.169) (size 0.5) (drill 0.3) (layers "F.Cu" "B.Cu") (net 1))
 (via (at 135.382 77.216) (size 0.5) (drill 0.3) (layers "F.Cu" "B.Cu") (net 1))
 (via (at 131.826 76.454) (size 0.5) (drill 0.3) (layers "F.Cu" "B.Cu") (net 1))
 (segment (start 135.509 89.41) (end 135.509 90.17) (width 0.25) (layer "F.Cu") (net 3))
 (segment (start 136.6038 80.6196) (end 135.9916 80.6196) (width 0.25) (layer "F.Cu") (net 3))
 (segment (start 130.81 80.01) (end 131.318 79.502) (width 0.25) (layer "F.Cu") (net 3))
 (segment (start 131.87 79.458) (end 131.87 78.4575) (width 0.25) (layer "F.Cu") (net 3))
 (segment (start 131.318 79.502) (end 131.826 79.502) (width 0.25) (layer "F.Cu") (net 3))
 (segment (start 131.782 77.045) (end 131.87 77.133) (width 0.25) (layer "F.Cu") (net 3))
 (segment (start 131.87 77.133) (end 131.87 78.4575) (width 0.25) (layer "F.Cu") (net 3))
 (segment (start 135.9916 80.6196) (end 135.87 80.498) (width 0.25) (layer "F.Cu") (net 3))
 (segment (start 130.81 80.419) (end 130.81 80.01) (width 0.25) (layer "F.Cu") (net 3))
 (segment (start 130.4575 77.045) (end 131.782 77.045) (width 0.25) (layer "F.Cu") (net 3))
 (segment (start 135.87 80.498) (end 135.87 78.4575) (width 0.25) (layer "F.Cu") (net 3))
 (segment (start 131.826 79.502) (end 131.87 79.458) (width 0.25) (layer "F.Cu") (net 3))
 (via (at 135.509 90.17) (size 0.5) (drill 0.3) (layers "F.Cu" "B.Cu") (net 3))
 (segment (start 127 53.34) (end 128.7525 53.34) (width 0.25) (layer "B.Cu") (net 3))
 (segment (start 128.7525 53.34) (end 130.6125 55.2) (width 0.25) (layer "B.Cu") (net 3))
 (segment (start 132.08 86.741) (end 131.953 86.614) (width 0.25) (layer "F.Cu") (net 5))
 (segment (start 131.953 86.614) (end 131.953 85.725) (width 0.25) (layer "F.Cu") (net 5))
 (segment (start 133.87 78.4575) (end 133.87 82.3898) (width 0.25) (layer "F.Cu") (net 5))
 (segment (start 131.953 85.725) (end 132.262 85.416) (width 0.25) (layer "F.Cu") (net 5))
 (segment (start 133.87 82.3898) (end 132.262 83.9978) (width 0.25) (layer "F.Cu") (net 5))
 (segment (start 132.362 86.741) (end 132.08 86.741) (width 0.25) (layer "F.Cu") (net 5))
 (segment (start 132.262 85.416) (end 132.262 83.9978) (width 0.25) (layer "F.Cu") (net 5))
 (segment (start 134.37 82.4058) (end 135.962 83.9978) (width 0.25) (layer "F.Cu") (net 2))
 (segment (start 134.37 78.4575) (end 134.37 82.4058) (width 0.25) (layer "F.Cu") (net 2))
 (segment (start 135.962 85.416) (end 135.962 83.9978) (width 0.25) (layer "F.Cu") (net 2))
 (segment (start 136.144 86.741) (end 136.271 86.614) (width 0.25) (layer "F.Cu") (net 2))
 (segment (start 136.271 85.725) (end 135.962 85.416) (width 0.25) (layer "F.Cu") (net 2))
 (segment (start 136.271 86.614) (end 136.271 85.725) (width 0.25) (layer "F.Cu") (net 2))
 (segment (start 135.862 86.741) (end 136.144 86.741) (width 0.25) (layer "F.Cu") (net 2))
 (segment (start 138.811 59.346) (end 136.665 57.2) (width 0.25) (layer "B.Cu") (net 11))
 (segment (start 136.665 57.2) (end 136.6125 57.2) (width 0.25) (layer "B.Cu") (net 11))
 (segment (start 137.705 68.58) (end 136.017 68.58) (width 0.25) (layer "B.Cu") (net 15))
 (segment (start 131.6125 58.166) (end 131.6125 56.2) (width 0.25) (layer "B.Cu") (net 15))
 (segment (start 131.826 58.3795) (end 131.6125 58.166) (width 0.25) (layer "B.Cu") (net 15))
 (segment (start 136.017 68.58) (end 131.826 64.389) (width 0.25) (layer "B.Cu") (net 15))
 (segment (start 131.826 64.389) (end 131.826 58.3795) (width 0.25) (layer "B.Cu") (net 15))
 (segment (start 131.6125 56.2) (end 132.6125 55.2) (width 0.25) (layer "B.Cu") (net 15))
 (segment (start 135.6125 58.0155) (end 135.6125 56.2) (width 0.25) (layer "B.Cu") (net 12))
 (segment (start 136.017 59.346) (end 136.017 58.42) (width 0.25) (layer "B.Cu") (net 12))
 (segment (start 135.6125 56.2) (end 136.6125 55.2) (width 0.25) (layer "B.Cu") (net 12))
 (segment (start 136.017 58.42) (end 135.6125 58.0155) (width 0.25) (layer "B.Cu") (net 12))
 (segment (start 130.429 57.3835) (end 130.6125 57.2) (width 0.25) (layer "B.Cu") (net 16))
 (segment (start 130.429 59.346) (end 130.429 57.3835) (width 0.25) (layer "B.Cu") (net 16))
 (segment (start 133.223 58.5895) (end 134.6125 57.2) (width 0.25) (layer "B.Cu") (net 13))
 (segment (start 133.223 59.346) (end 133.223 58.5895) (width 0.25) (layer "B.Cu") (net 13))
 (segment (start 129.413 80.389) (end 129.413 80.01) (width 0.25) (layer "F.Cu") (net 8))
 (segment (start 129.413 80.01) (end 129.921 79.502) (width 0.25) (layer "F.Cu") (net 8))
 (segment (start 131.56 75.045) (end 131.572 75.057) (width 0.25) (layer "F.Cu") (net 8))
 (segment (start 130.4575 75.045) (end 131.56 75.045) (width 0.25) (layer "F.Cu") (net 8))
 (via (at 129.921 79.502) (size 0.5) (drill 0.3) (layers "F.Cu" "B.Cu") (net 8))
 (via (at 131.572 75.057) (size 0.5) (drill 0.3) (layers "F.Cu" "B.Cu") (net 8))
 (segment (start 131.572 75.057) (end 129.921 76.708) (width 0.25) (layer "B.Cu") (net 8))
 (segment (start 129.921 76.708) (end 129.921 77.978) (width 0.25) (layer "B.Cu") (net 8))
 (segment (start 129.921 77.978) (end 129.921 79.502) (width 0.25) (layer "B.Cu") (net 8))
 (segment (start 134.87 78.4575) (end 134.87 79.6815) (width 0.25) (layer "F.Cu") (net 4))
 (segment (start 135.509 88.39) (end 135.509 88.011) (width 0.25) (layer "F.Cu") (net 4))
 (segment (start 135.382 87.884) (end 134.874 87.884) (width 0.25) (layer "F.Cu") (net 4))
 (segment (start 134.239 87.884) (end 134.239 88.42) (width 0.25) (layer "F.Cu") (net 4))
 (segment (start 135.509 88.011) (end 135.382 87.884) (width 0.25) (layer "F.Cu") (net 4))
 (segment (start 134.874 87.884) (end 134.239 87.884) (width 0.25) (layer "F.Cu") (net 4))
 (segment (start 134.87 79.6815) (end 134.9445 79.756) (width 0.25) (layer "F.Cu") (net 4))
 (via (at 134.9445 79.756) (size 0.5) (drill 0.3) (layers "F.Cu" "B.Cu") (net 4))
 (via (at 134.874 87.884) (size 0.5) (drill 0.3) (layers "F.Cu" "B.Cu") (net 4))
 (segment (start 134.9445 87.122) (end 134.9445 87.5595) (width 0.25) (layer "B.Cu") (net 4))
 (segment (start 134.9445 79.756) (end 134.9445 87.122) (width 0.25) (layer "B.Cu") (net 4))
 (segment (start 134.9445 87.8135) (end 134.874 87.884) (width 0.25) (layer "B.Cu") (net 4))
 (segment (start 134.9445 87.122) (end 134.9445 87.8135) (width 0.25) (layer "B.Cu") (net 4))
 (segment (start 130.4575 72.545) (end 129.441 72.545) (width 0.25) (layer "F.Cu") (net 45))
 (segment (start 128.397 71.501) (end 128.397 69.977) (width 0.25) (layer "F.Cu") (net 45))
 (segment (start 128.397 69.977) (end 127 68.58) (width 0.25) (layer "F.Cu") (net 45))
 (segment (start 129.441 72.545) (end 128.397 71.501) (width 0.25) (layer "F.Cu") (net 45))
 (segment (start 128.925 73.045) (end 127 71.12) (width 0.25) (layer "F.Cu") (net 46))
 (segment (start 130.4575 73.045) (end 128.925 73.045) (width 0.25) (layer "F.Cu") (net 46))
 (segment (start 130.4575 73.545) (end 127.115 73.545) (width 0.25) (layer "F.Cu") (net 47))
 (segment (start 127 73.66) (end 127 74.422) (width 0.25) (layer "F.Cu") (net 47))
 (segment (start 127.115 73.545) (end 127 73.66) (width 0.25) (layer "F.Cu") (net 47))
 (segment (start 127 76.708) (end 127 76.2) (width 0.25) (layer "F.Cu") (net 48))
 (segment (start 129.155 74.045) (end 127 76.2) (width 0.25) (layer "F.Cu") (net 48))
 (segment (start 130.4575 74.045) (end 129.155 74.045) (width 0.25) (layer "F.Cu") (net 48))
 (segment (start 129.291396 74.545) (end 130.4575 74.545) (width 0.25) (layer "F.Cu") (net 49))
 (segment (start 127 78.74) (end 128.27 77.47) (width 0.25) (layer "F.Cu") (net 49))
 (segment (start 128.27 75.566396) (end 129.291396 74.545) (width 0.25) (layer "F.Cu") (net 49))
 (segment (start 128.27 77.47) (end 128.27 75.566396) (width 0.25) (layer "F.Cu") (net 49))
 (segment (start 128.72 76.131) (end 128.72 79.56) (width 0.25) (layer "F.Cu") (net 50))
 (segment (start 130.4575 75.545) (end 129.306 75.545) (width 0.25) (layer "F.Cu") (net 50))
 (segment (start 128.72 79.56) (end 127 81.28) (width 0.25) (layer "F.Cu") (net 50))
 (segment (start 129.306 75.545) (end 128.72 76.131) (width 0.25) (layer "F.Cu") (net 50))
 (segment (start 129.2945 76.192896) (end 129.2945 77.724) (width 0.25) (layer "F.Cu") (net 51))
 (segment (start 130.4575 76.045) (end 129.442396 76.045) (width 0.25) (layer "F.Cu") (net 51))
 (segment (start 127.569874 83.82) (end 127 83.82) (width 0.25) (layer "F.Cu") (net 51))
 (segment (start 129.442396 76.045) (end 129.2945 76.192896) (width 0.25) (layer "F.Cu") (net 51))
 (via (at 129.2945 77.724) (size 0.5) (drill 0.3) (layers "F.Cu" "B.Cu") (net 51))
 (segment (start 129.2945 81.5255) (end 127 83.82) (width 0.25) (layer "B.Cu") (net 51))
 (segment (start 129.2945 77.724) (end 129.2945 81.5255) (width 0.25) (layer "B.Cu") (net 51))
 (segment (start 139.155 65.913) (end 142.113 65.913) (width 0.25) (layer "B.Cu") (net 22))
 (segment (start 142.113 65.913) (end 142.24 66.04) (width 0.25) (layer "B.Cu") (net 22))
 (segment (start 140.589 68.58) (end 140.716 68.58) (width 0.25) (layer "B.Cu") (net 23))
 (segment (start 139.155 68.58) (end 140.716 68.58) (width 0.25) (layer "B.Cu") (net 23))
 (segment (start 140.716 68.58) (end 142.24 68.58) (width 0.25) (layer "B.Cu") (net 23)))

